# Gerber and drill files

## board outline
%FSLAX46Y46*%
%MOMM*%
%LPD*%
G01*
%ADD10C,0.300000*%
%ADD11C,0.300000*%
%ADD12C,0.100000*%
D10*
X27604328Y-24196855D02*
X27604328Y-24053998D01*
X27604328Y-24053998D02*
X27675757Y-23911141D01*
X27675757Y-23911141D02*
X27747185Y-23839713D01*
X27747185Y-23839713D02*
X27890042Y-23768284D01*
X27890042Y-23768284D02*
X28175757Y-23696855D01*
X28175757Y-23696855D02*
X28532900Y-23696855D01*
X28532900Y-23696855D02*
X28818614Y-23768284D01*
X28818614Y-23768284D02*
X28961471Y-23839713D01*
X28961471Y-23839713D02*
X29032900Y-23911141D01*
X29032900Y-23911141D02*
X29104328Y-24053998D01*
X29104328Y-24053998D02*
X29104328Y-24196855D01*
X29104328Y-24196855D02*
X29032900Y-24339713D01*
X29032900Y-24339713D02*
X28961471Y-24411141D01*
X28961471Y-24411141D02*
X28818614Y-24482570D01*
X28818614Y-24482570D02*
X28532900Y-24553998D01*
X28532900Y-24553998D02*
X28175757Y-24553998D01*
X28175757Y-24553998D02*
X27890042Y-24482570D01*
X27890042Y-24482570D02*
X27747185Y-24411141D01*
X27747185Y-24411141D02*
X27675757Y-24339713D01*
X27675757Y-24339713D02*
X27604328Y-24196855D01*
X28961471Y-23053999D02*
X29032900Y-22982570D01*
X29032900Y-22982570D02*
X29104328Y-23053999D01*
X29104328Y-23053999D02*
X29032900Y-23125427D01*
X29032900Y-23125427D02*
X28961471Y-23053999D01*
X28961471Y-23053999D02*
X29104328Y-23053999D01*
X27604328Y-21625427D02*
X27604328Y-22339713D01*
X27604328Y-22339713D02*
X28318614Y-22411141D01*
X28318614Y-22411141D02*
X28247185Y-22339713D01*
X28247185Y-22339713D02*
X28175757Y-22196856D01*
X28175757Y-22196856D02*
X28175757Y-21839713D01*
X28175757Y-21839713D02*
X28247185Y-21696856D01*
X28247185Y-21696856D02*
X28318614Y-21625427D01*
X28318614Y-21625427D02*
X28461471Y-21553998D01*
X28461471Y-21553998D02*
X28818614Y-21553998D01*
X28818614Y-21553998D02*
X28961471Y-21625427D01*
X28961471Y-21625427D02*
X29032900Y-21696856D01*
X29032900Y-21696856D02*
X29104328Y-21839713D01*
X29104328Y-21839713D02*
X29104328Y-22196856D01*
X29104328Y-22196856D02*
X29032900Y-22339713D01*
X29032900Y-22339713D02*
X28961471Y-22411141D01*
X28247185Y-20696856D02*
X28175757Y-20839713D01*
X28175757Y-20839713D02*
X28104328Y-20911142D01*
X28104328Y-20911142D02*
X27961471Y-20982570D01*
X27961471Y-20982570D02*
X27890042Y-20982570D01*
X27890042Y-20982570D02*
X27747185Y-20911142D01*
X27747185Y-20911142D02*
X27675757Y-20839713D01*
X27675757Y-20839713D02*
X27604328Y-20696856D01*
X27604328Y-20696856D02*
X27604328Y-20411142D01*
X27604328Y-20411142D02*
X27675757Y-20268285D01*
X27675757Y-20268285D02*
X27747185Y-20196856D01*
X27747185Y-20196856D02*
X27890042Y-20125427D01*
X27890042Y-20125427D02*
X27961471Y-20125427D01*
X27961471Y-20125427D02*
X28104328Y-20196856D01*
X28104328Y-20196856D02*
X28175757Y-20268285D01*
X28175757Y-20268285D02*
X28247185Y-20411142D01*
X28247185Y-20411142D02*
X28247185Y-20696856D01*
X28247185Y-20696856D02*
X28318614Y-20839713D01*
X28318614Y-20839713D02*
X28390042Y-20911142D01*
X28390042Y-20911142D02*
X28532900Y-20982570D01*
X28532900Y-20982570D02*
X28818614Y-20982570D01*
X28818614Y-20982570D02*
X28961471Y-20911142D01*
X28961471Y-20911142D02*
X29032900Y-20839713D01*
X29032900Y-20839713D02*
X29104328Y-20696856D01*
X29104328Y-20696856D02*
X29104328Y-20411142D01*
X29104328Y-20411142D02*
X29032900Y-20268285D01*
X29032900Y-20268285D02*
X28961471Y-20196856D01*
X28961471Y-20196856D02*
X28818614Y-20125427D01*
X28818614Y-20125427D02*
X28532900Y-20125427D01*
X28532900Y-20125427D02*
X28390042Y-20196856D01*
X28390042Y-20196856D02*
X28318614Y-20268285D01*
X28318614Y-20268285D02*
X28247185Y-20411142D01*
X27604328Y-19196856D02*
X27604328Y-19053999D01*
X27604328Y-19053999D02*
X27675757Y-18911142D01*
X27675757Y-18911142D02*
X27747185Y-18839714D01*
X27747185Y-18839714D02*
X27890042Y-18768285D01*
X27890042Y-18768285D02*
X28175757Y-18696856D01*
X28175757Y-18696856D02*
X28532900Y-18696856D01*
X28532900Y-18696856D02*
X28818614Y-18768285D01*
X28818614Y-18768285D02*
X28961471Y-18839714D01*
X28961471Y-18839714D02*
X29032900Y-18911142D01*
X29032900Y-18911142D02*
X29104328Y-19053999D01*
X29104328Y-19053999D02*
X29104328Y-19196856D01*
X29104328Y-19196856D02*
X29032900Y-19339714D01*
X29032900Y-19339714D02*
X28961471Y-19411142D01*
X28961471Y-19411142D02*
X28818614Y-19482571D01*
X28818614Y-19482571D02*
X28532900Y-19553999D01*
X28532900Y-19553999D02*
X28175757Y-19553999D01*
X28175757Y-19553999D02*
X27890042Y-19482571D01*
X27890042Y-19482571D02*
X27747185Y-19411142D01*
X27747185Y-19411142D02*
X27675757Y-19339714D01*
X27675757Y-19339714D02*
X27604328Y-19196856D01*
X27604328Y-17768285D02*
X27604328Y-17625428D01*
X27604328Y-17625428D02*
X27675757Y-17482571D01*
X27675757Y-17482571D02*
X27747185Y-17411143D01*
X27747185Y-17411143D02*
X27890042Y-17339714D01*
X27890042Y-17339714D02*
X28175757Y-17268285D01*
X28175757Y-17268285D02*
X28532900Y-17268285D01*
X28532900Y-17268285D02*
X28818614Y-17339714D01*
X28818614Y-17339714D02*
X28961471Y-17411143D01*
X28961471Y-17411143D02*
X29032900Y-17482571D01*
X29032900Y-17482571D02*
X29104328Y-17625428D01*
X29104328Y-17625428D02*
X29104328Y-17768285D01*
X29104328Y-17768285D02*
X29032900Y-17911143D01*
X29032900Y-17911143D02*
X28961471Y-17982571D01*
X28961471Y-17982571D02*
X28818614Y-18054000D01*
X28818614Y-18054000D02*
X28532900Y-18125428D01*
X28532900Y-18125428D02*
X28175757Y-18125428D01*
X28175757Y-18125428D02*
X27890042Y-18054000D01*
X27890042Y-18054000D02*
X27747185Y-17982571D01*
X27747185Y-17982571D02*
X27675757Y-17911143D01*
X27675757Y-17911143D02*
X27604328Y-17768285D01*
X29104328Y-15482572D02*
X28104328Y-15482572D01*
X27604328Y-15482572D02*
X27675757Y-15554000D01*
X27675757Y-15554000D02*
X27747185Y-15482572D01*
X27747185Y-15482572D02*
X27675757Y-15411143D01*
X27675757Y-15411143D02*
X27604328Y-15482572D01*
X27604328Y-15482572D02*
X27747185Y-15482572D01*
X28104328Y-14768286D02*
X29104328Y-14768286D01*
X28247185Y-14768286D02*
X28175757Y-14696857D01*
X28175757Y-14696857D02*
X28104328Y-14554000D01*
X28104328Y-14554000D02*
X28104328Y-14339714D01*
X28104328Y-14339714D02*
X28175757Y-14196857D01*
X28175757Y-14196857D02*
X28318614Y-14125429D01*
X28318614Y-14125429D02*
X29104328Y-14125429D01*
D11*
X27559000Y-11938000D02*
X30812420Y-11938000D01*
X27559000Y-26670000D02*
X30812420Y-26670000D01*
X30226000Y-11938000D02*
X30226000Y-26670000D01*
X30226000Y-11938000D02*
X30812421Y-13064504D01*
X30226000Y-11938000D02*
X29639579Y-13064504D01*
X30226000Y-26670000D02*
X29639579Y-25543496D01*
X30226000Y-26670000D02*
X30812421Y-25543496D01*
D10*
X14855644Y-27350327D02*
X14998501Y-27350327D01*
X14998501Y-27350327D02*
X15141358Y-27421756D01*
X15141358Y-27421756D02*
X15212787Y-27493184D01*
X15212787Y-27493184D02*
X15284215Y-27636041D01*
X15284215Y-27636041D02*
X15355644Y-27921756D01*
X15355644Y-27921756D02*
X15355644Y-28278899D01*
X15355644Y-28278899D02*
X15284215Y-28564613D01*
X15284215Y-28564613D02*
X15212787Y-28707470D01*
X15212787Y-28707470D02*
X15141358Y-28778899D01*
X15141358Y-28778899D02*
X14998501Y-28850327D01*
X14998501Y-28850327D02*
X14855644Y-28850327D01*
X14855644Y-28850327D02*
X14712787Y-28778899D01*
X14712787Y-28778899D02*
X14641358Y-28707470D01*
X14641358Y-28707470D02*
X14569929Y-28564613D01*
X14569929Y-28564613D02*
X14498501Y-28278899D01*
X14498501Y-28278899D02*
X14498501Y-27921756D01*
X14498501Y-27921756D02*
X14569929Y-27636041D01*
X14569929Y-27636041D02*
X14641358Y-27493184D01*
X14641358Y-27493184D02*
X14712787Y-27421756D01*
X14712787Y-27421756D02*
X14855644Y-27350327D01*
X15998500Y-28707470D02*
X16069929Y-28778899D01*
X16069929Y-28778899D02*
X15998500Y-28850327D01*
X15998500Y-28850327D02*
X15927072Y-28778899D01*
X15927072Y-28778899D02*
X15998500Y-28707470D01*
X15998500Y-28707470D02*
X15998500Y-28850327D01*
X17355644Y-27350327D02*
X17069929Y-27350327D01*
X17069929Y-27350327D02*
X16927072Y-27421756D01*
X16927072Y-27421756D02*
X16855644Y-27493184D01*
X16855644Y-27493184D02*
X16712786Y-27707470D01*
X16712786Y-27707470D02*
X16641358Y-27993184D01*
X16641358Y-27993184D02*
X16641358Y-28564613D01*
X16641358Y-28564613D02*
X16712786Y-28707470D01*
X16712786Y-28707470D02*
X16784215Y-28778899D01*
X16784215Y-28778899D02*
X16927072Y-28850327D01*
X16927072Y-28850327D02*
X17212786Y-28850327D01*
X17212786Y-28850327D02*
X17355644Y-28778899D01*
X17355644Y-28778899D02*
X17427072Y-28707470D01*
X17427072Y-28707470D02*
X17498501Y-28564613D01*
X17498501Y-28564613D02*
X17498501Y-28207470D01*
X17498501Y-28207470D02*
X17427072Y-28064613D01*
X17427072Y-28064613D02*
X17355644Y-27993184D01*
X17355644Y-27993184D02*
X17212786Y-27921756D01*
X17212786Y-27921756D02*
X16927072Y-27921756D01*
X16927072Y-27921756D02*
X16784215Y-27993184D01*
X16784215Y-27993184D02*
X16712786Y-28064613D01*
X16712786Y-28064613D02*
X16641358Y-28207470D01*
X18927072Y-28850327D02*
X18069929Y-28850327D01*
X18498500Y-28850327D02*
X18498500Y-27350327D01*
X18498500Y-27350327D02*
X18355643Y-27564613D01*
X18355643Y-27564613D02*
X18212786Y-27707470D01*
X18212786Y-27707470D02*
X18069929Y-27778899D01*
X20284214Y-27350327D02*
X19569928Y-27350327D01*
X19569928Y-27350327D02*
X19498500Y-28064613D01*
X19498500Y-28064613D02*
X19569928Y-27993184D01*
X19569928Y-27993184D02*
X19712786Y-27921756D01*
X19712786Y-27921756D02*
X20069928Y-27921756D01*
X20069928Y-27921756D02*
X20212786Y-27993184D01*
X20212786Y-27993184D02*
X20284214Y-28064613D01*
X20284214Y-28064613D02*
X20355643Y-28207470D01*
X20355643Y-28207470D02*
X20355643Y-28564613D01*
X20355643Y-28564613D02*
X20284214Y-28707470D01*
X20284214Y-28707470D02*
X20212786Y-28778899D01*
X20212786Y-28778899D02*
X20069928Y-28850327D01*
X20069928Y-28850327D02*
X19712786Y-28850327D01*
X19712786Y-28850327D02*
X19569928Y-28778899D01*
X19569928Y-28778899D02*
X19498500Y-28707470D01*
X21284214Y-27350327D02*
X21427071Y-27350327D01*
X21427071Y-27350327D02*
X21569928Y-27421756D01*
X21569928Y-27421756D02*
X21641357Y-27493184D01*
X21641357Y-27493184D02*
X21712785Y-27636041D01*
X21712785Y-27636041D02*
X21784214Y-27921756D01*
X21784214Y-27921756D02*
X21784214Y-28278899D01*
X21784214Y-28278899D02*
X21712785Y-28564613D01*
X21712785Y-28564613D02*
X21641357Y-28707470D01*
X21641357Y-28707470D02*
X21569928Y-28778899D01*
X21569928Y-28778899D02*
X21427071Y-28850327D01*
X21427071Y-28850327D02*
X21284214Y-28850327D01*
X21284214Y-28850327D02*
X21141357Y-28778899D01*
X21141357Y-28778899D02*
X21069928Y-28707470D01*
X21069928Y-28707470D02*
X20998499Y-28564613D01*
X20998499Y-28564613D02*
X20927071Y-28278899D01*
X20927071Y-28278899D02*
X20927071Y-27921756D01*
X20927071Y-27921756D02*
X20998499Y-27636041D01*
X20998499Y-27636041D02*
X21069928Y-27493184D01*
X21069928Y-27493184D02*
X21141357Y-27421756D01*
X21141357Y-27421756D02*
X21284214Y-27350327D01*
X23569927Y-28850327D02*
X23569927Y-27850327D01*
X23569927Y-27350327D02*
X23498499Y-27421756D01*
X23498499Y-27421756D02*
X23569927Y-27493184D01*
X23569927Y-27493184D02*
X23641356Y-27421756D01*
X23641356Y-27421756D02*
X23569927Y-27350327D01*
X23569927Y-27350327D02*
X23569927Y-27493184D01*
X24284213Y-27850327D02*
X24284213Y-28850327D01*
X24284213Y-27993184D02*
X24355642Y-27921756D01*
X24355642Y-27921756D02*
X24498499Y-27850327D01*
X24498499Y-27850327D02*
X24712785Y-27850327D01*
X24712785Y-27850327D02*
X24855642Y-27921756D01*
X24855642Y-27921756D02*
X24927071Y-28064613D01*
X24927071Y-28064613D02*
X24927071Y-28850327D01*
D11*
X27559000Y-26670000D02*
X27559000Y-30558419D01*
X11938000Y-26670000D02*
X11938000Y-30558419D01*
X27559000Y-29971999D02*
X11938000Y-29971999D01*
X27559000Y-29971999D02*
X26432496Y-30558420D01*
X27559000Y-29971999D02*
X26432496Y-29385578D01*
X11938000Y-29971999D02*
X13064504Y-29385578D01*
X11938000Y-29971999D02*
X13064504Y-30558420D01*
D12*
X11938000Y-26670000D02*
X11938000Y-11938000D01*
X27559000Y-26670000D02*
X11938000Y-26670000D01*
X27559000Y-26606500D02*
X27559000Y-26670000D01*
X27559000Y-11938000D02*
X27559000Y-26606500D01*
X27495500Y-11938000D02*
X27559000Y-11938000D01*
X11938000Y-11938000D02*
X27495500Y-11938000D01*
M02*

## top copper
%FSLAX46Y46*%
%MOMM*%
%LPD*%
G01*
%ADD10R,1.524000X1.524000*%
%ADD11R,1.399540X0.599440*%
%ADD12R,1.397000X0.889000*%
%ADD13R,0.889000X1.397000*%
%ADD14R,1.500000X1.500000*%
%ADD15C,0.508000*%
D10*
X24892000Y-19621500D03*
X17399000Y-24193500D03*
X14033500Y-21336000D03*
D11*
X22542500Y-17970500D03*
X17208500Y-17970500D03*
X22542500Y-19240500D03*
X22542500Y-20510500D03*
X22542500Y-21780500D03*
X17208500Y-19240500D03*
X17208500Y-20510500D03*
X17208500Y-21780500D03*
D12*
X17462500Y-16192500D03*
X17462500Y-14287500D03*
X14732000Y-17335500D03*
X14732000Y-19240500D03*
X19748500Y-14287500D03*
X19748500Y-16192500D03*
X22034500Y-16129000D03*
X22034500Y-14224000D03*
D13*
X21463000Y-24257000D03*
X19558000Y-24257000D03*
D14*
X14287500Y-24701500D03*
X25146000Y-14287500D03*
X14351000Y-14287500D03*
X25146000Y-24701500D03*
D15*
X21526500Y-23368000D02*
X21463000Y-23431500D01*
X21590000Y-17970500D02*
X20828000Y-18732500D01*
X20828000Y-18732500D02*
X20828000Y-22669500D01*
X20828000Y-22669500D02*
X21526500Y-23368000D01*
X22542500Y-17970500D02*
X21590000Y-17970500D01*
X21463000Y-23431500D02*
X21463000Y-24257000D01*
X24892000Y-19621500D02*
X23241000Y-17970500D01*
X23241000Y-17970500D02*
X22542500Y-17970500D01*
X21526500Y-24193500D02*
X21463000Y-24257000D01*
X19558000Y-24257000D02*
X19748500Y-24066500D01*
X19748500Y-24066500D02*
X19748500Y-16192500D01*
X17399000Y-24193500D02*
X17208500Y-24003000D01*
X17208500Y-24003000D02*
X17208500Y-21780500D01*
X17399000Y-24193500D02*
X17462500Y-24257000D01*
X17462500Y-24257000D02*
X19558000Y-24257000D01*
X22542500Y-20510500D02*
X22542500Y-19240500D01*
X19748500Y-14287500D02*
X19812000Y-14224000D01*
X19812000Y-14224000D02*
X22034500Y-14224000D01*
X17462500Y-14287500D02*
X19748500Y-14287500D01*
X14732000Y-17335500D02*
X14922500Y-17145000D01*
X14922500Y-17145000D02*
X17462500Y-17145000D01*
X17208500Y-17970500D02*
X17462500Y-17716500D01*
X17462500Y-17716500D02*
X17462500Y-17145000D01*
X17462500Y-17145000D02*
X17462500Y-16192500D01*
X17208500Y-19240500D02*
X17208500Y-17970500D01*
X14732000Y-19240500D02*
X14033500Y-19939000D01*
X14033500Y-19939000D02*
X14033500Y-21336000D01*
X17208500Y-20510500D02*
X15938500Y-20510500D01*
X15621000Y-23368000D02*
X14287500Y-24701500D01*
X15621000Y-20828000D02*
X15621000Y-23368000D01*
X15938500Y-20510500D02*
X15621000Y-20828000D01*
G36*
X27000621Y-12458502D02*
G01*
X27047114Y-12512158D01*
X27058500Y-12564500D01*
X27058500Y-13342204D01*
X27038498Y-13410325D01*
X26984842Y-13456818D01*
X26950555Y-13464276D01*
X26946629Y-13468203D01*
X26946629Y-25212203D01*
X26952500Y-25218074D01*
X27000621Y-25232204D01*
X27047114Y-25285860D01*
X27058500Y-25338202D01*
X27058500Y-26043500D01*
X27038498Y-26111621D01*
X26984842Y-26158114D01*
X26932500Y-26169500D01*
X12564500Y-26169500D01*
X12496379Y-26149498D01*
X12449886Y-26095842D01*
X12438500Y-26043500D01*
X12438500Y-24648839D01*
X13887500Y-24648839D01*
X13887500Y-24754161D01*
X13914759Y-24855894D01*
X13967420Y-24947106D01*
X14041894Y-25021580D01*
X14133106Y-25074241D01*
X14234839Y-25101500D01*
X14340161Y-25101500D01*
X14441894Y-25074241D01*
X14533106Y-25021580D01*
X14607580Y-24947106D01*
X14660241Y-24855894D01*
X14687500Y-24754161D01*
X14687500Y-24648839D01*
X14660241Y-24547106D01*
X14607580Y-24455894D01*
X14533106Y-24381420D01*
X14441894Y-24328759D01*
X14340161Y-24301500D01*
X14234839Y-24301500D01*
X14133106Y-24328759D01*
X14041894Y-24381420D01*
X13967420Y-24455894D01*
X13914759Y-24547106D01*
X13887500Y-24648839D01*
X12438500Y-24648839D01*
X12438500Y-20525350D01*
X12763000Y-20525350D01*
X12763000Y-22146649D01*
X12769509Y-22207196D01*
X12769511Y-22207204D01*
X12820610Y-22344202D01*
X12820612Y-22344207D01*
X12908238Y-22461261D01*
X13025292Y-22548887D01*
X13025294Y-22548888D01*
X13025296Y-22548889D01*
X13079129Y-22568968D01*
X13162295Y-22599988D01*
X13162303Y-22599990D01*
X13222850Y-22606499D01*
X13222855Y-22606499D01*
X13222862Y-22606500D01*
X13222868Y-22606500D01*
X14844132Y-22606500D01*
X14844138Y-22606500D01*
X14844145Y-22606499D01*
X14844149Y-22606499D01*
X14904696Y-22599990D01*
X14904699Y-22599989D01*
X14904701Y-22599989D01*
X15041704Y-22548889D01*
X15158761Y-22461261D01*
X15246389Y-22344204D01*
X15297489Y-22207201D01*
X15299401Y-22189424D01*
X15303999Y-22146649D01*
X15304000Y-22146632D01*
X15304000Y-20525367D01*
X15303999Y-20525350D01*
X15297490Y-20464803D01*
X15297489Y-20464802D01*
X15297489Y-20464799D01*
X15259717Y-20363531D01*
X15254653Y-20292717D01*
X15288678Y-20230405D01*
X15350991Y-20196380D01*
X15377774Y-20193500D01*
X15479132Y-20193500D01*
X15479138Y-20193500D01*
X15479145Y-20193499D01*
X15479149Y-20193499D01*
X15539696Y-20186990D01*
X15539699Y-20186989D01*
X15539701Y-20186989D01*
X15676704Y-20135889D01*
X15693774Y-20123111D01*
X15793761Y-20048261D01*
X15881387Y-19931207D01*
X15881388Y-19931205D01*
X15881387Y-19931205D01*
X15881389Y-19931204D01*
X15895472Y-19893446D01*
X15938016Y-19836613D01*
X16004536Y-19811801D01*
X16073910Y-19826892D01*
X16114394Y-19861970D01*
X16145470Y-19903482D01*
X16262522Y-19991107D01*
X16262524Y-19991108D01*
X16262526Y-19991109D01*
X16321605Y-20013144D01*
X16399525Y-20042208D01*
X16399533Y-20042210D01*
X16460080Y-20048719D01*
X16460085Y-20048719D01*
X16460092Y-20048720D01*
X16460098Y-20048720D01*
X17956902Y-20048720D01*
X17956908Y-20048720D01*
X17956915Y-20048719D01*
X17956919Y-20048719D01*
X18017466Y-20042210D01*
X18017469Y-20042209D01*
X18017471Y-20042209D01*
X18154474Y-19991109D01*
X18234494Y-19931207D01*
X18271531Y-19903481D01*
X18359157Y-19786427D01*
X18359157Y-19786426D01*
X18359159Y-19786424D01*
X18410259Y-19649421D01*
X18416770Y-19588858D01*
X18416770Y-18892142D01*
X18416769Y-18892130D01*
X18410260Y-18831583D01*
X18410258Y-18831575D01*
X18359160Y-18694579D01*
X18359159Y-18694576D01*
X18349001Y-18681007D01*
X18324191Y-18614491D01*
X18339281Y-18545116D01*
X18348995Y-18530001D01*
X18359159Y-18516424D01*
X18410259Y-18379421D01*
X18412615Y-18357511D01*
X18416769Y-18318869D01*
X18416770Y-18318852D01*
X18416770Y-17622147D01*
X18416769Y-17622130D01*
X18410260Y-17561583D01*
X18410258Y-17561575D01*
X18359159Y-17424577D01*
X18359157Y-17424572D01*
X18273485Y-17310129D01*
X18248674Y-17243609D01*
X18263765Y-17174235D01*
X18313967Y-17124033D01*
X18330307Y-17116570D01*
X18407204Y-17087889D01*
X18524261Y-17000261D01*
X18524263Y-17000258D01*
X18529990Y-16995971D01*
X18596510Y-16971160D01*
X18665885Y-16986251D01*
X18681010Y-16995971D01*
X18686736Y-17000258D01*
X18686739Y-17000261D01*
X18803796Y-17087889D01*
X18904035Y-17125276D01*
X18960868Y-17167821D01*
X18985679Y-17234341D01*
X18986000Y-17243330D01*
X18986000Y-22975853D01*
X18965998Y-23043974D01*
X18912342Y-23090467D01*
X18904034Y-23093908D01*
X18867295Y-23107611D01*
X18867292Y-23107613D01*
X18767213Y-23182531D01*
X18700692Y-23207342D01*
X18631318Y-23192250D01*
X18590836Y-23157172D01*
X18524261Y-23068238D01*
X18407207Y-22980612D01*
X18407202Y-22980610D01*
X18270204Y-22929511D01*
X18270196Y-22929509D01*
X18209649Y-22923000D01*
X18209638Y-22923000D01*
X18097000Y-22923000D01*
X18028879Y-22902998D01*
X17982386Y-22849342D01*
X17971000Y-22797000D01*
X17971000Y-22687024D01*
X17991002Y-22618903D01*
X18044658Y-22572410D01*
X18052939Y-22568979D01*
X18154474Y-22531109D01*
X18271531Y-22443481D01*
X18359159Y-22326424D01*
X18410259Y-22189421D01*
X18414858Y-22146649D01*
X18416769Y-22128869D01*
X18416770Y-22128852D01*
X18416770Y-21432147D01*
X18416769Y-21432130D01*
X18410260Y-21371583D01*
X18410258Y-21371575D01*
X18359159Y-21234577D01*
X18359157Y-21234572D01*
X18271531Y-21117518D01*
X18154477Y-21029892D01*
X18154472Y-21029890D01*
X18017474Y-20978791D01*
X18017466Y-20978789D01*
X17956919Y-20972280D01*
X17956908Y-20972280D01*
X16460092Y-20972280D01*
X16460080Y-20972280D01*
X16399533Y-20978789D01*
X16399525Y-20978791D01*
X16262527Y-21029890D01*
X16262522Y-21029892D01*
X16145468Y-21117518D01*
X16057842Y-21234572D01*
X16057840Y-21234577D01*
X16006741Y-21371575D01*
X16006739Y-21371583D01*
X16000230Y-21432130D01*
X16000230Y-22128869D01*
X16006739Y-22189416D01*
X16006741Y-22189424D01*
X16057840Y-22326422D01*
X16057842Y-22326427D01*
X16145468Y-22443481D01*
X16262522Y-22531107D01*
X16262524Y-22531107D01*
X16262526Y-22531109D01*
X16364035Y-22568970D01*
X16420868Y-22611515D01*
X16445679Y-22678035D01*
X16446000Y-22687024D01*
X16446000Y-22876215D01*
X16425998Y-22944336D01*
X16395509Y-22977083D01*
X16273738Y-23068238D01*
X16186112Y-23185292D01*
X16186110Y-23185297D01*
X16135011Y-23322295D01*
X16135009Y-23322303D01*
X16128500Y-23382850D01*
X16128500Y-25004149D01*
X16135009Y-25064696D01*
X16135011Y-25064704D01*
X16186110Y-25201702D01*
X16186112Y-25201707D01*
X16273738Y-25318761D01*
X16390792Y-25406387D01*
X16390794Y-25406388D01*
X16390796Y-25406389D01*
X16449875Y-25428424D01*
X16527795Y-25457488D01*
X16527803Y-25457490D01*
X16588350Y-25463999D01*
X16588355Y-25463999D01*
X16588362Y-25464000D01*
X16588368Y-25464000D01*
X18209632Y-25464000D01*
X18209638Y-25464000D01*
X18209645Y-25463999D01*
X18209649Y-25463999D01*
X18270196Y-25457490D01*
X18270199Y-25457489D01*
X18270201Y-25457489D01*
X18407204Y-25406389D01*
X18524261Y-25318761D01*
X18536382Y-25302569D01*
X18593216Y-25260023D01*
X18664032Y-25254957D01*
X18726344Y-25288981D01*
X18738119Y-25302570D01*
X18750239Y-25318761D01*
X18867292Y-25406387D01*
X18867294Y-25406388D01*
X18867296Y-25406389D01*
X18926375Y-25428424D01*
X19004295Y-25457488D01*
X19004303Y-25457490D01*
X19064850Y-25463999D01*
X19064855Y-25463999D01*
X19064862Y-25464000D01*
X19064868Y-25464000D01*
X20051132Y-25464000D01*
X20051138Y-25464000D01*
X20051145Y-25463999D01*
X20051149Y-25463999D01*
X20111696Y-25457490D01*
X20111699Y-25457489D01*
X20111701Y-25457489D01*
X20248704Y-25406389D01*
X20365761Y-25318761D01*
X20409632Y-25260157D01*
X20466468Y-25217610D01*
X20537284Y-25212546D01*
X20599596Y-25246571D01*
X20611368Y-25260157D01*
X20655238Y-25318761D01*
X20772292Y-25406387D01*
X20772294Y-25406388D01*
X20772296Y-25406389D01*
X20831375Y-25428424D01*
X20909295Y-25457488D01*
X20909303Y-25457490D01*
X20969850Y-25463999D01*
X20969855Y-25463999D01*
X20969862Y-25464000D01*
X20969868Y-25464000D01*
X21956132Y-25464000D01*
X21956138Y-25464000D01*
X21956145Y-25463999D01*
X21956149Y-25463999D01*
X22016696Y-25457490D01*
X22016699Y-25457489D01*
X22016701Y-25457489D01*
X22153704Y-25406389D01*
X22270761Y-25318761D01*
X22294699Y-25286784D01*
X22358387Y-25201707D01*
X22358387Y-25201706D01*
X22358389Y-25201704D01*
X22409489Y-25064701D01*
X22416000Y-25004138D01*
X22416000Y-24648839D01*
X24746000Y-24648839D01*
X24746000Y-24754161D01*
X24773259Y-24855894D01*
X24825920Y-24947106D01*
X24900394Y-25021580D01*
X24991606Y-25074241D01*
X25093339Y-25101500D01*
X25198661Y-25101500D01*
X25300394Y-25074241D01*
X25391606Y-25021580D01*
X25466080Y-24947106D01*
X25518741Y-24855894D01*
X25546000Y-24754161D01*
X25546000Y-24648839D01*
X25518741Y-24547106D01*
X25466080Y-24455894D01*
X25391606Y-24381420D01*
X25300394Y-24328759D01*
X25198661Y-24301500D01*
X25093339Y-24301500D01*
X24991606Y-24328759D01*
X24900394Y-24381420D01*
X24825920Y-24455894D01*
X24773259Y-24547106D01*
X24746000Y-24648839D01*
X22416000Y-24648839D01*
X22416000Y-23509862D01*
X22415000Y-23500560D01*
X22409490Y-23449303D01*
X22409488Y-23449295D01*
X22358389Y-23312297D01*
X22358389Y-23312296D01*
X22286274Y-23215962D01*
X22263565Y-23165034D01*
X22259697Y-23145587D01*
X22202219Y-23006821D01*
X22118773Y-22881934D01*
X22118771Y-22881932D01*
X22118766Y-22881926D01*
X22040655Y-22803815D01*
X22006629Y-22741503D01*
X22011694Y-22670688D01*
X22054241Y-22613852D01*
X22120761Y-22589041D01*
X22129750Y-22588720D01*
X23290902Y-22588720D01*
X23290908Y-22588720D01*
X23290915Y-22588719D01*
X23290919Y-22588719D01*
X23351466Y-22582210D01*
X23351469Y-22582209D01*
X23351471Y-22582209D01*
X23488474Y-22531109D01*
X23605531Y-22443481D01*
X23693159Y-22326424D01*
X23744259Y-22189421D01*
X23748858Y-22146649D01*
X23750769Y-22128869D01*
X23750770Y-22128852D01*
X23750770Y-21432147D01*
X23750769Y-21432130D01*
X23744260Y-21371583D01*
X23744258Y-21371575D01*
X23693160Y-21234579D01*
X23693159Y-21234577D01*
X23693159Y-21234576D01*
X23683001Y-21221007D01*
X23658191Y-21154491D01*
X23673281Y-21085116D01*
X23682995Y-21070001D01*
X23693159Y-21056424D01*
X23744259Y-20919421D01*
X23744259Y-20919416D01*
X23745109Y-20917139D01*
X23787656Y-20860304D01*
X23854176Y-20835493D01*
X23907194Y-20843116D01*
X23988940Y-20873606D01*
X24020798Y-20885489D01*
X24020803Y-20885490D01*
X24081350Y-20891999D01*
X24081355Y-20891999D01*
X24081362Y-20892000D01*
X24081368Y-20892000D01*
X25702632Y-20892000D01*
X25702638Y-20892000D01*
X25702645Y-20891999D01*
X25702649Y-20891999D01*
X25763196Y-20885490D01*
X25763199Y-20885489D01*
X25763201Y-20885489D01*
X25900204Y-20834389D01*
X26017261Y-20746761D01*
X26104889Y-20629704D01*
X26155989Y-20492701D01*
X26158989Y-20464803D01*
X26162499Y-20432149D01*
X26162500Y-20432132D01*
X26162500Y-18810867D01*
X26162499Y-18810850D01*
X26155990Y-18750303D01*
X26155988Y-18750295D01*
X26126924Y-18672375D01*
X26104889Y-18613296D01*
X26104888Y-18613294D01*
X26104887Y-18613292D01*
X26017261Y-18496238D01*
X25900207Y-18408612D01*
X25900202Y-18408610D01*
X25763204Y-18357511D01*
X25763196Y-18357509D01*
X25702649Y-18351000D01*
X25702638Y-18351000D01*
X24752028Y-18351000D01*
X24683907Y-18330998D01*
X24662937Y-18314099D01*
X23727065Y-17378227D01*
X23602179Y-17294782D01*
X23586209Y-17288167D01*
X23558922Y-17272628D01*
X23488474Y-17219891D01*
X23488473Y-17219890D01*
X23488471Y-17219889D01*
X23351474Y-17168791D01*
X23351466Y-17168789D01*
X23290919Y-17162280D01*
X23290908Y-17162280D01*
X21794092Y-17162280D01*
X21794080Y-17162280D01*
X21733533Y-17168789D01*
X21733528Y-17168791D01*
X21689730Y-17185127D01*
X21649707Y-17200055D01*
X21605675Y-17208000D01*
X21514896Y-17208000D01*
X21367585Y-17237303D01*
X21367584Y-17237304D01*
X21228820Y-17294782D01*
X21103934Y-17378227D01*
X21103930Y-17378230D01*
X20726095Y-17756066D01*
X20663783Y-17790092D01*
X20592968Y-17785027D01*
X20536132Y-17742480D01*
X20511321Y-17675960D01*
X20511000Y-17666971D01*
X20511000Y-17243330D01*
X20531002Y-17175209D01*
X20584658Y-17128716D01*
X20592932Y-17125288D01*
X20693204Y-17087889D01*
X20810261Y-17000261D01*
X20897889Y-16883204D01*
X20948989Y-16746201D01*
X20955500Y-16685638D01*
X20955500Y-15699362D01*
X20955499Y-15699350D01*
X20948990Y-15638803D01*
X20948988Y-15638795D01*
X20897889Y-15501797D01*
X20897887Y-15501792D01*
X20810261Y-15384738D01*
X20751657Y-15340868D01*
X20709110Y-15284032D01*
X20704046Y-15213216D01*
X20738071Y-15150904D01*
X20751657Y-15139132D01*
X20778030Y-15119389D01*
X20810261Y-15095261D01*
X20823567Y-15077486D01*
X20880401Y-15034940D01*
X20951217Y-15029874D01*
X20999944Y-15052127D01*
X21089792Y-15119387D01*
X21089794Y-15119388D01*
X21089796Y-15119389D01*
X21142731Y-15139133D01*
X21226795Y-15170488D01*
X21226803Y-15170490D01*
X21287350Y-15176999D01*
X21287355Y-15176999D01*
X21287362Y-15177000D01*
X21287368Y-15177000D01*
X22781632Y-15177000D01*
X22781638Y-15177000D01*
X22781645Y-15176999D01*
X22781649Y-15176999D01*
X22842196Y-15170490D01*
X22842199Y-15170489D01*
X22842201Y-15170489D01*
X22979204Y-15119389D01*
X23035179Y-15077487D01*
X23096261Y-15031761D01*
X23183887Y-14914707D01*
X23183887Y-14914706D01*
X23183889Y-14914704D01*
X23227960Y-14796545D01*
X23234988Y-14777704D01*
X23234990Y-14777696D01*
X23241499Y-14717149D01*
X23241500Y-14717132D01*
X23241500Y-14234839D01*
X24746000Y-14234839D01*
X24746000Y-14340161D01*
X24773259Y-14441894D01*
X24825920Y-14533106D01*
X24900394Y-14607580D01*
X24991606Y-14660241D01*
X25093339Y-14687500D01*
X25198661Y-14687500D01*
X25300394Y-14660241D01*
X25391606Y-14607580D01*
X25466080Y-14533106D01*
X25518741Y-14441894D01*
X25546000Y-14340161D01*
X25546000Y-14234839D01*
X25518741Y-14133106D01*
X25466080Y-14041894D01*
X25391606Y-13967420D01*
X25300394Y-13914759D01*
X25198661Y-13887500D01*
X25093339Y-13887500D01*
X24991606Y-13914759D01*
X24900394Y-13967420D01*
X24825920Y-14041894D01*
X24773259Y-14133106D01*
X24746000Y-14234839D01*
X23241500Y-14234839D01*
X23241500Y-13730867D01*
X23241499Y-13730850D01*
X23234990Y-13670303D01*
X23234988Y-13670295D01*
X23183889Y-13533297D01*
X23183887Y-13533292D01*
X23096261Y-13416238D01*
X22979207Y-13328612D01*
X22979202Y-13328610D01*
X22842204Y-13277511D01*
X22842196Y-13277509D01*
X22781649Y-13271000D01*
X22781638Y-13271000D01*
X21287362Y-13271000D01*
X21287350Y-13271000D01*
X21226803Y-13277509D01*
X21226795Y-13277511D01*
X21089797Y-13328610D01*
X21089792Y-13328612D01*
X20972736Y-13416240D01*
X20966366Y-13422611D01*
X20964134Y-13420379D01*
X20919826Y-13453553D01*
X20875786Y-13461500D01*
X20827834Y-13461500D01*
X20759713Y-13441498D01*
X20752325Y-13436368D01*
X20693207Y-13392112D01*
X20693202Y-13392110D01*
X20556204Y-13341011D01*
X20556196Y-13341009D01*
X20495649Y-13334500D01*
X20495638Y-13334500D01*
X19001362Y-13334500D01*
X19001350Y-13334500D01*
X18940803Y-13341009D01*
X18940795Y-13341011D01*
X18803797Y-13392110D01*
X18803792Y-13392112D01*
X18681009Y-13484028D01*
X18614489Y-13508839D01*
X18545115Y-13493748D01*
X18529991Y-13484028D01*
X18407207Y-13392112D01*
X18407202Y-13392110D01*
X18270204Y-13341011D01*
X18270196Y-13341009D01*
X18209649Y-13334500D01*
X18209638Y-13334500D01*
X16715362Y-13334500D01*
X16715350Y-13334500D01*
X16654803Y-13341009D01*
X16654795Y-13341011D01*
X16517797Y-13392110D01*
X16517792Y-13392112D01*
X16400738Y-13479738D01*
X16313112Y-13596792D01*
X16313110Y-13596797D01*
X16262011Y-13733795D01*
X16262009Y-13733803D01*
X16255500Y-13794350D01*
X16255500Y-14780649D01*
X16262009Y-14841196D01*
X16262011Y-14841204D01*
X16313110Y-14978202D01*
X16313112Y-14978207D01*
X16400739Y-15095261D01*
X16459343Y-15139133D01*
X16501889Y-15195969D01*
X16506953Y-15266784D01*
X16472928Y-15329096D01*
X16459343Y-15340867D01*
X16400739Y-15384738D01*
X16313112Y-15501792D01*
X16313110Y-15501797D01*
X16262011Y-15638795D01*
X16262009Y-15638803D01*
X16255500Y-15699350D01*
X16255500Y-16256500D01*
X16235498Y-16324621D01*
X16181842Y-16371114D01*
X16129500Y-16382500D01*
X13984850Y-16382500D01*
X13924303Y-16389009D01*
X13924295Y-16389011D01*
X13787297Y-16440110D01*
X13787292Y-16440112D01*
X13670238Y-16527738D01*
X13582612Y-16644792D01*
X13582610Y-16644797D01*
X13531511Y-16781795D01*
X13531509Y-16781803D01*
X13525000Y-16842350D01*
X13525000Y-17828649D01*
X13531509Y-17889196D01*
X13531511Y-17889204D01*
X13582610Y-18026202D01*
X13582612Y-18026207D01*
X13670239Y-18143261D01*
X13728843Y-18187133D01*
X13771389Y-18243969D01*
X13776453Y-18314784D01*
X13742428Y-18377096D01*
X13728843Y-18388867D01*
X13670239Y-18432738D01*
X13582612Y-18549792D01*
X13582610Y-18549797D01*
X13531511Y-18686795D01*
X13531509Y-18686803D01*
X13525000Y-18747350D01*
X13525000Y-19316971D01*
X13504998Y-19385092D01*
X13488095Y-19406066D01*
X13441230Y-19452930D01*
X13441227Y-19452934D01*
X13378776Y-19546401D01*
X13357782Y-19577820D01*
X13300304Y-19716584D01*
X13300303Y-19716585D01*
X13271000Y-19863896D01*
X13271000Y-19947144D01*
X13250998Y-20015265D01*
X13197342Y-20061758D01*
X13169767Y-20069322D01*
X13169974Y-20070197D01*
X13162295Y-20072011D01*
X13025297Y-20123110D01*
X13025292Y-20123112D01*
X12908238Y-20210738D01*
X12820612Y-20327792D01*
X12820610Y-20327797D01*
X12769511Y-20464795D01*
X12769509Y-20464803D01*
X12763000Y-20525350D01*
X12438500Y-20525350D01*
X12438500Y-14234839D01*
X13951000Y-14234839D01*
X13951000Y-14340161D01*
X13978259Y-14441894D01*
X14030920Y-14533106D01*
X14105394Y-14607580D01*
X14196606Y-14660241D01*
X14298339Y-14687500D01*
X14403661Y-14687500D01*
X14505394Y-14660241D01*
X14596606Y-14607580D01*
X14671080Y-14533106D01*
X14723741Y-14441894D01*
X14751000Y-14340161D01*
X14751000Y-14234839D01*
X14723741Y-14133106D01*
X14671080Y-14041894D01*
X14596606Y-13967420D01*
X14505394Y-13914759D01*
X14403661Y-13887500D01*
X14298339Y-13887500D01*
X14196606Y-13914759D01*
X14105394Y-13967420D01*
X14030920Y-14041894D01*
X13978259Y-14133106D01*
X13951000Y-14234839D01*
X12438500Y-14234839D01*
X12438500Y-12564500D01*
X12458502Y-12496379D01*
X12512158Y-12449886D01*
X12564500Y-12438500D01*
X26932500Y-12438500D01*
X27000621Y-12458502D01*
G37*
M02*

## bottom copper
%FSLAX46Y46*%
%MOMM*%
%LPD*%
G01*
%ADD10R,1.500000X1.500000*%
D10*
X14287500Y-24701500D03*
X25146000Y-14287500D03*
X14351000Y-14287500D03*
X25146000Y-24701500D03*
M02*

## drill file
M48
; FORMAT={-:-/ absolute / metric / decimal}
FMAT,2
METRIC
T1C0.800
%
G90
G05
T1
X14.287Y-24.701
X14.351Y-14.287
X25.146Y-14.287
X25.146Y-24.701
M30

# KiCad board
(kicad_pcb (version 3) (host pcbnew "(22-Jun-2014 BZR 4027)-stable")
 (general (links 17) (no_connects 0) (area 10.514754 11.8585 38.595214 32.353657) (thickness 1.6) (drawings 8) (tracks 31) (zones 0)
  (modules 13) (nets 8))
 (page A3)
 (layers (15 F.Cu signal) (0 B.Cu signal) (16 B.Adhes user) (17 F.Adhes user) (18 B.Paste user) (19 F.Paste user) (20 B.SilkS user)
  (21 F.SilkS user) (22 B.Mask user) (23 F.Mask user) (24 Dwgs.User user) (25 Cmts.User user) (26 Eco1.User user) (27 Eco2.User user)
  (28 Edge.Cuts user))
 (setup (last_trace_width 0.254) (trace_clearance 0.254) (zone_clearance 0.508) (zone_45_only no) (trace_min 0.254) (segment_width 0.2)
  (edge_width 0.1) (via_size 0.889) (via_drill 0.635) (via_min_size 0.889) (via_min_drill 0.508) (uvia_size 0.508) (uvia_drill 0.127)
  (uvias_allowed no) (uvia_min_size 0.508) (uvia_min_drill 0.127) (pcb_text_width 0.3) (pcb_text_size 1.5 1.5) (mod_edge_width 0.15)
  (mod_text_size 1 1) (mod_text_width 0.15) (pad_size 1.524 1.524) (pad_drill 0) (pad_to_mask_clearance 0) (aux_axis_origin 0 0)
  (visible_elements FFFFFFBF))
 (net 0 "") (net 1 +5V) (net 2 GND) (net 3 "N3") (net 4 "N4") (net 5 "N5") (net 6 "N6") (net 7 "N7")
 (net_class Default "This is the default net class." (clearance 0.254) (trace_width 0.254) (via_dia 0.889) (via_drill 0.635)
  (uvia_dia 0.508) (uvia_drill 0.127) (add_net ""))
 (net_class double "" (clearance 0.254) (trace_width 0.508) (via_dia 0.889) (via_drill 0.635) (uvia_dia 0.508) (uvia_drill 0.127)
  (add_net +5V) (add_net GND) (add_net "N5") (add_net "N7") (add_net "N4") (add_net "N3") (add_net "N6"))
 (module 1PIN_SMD (layer F.Cu) (at 24.892 19.6215)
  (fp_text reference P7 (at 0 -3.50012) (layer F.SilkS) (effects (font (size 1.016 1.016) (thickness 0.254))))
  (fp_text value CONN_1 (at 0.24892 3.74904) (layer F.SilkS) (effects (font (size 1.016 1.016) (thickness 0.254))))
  (pad 1 smd rect (at 0 0) (size 1.524 1.524) (layers F.Cu F.Paste F.SilkS F.Mask) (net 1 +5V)))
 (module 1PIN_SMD (layer F.Cu) (at 17.399 24.1935)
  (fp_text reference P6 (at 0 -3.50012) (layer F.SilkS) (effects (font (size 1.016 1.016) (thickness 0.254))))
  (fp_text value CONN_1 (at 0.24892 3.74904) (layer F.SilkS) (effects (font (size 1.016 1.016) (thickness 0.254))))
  (pad 1 smd rect (at 0 0) (size 1.524 1.524) (layers F.Cu F.Paste F.SilkS F.Mask) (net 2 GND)))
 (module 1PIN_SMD (layer F.Cu) (at 14.0335 21.336)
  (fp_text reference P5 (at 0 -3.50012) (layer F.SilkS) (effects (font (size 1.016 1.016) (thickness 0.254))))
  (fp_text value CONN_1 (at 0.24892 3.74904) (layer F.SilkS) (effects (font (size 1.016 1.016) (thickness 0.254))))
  (pad 1 smd rect (at 0 0) (size 1.524 1.524) (layers F.Cu F.Paste F.SilkS F.Mask) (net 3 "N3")))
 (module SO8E (layer F.Cu) (at 19.8755 19.8755 270)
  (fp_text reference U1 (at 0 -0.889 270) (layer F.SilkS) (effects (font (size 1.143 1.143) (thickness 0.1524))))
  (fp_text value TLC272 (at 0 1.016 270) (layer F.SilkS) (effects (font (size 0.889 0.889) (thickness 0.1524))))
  (pad 8 smd rect (at -1.905 -2.667 270) (size 0.59944 1.39954) (layers F.Cu F.Paste F.Mask) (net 1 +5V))
  (pad 1 smd rect (at -1.905 2.667 270) (size 0.59944 1.39954) (layers F.Cu F.Paste F.Mask) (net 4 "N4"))
  (pad 7 smd rect (at -0.635 -2.667 270) (size 0.59944 1.39954) (layers F.Cu F.Paste F.Mask) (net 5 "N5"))
  (pad 6 smd rect (at 0.635 -2.667 270) (size 0.59944 1.39954) (layers F.Cu F.Paste F.Mask) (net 5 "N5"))
  (pad 5 smd rect (at 1.905 -2.667 270) (size 0.59944 1.39954) (layers F.Cu F.Paste F.Mask))
  (pad 2 smd rect (at -0.635 2.667 270) (size 0.59944 1.39954) (layers F.Cu F.Paste F.Mask) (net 4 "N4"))
  (pad 3 smd rect (at 0.635 2.667 270) (size 0.59944 1.39954) (layers F.Cu F.Paste F.Mask) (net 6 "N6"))
  (pad 4 smd rect (at 1.905 2.667 270) (size 0.59944 1.39954) (layers F.Cu F.Paste F.Mask) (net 2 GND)))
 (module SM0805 (layer F.Cu) (at 17.4625 15.24 90)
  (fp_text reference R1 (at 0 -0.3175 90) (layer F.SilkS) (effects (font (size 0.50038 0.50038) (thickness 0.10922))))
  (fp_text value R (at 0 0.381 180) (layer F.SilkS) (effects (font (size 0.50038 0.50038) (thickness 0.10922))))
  (pad 1 smd rect (at -0.9525 0 90) (size 0.889 1.397) (layers F.Cu F.Paste F.Mask) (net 4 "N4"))
  (pad 2 smd rect (at 0.9525 0 90) (size 0.889 1.397) (layers F.Cu F.Paste F.Mask) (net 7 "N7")))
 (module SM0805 (layer F.Cu) (at 14.732 18.288 270)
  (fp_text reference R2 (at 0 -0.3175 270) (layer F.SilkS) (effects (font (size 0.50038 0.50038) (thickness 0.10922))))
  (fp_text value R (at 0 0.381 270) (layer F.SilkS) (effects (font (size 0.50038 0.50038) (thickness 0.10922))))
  (pad 1 smd rect (at -0.9525 0 270) (size 0.889 1.397) (layers F.Cu F.Paste F.Mask) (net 4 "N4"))
  (pad 2 smd rect (at 0.9525 0 270) (size 0.889 1.397) (layers F.Cu F.Paste F.Mask) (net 3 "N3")))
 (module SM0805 (layer F.Cu) (at 19.7485 15.24 270)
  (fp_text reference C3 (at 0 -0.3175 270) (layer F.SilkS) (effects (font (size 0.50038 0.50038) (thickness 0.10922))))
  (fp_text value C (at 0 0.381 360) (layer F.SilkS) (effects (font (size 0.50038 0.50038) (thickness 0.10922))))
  (pad 1 smd rect (at -0.9525 0 270) (size 0.889 1.397) (layers F.Cu F.Paste F.Mask) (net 7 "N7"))
  (pad 2 smd rect (at 0.9525 0 270) (size 0.889 1.397) (layers F.Cu F.Paste F.Mask) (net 2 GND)))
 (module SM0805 (layer F.Cu) (at 22.0345 15.1765 90)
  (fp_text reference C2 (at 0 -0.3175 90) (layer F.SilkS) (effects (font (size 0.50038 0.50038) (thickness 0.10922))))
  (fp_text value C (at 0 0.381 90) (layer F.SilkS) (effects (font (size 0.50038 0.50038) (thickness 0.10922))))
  (pad 1 smd rect (at -0.9525 0 90) (size 0.889 1.397) (layers F.Cu F.Paste F.Mask) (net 6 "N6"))
  (pad 2 smd rect (at 0.9525 0 90) (size 0.889 1.397) (layers F.Cu F.Paste F.Mask) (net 7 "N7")))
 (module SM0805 (layer F.Cu) (at 20.5105 24.257 180)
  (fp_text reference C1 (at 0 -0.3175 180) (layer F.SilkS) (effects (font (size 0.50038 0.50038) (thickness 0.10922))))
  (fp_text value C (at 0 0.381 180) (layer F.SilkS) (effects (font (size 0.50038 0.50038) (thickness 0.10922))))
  (pad 1 smd rect (at -0.9525 0 180) (size 0.889 1.397) (layers F.Cu F.Paste F.Mask) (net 1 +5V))
  (pad 2 smd rect (at 0.9525 0 180) (size 0.889 1.397) (layers F.Cu F.Paste F.Mask) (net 2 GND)))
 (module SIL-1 (layer F.Cu) (at 14.2875 24.7015)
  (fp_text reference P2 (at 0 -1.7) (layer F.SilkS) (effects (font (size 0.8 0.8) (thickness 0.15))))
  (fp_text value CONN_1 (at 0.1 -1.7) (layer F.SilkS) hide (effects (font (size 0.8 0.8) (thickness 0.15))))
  (pad 1 thru_hole rect (at 0 0) (size 1.5 1.5) (drill 0.8) (layers *.Cu *.Mask F.SilkS) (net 6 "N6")))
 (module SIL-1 (layer F.Cu) (at 25.146 14.2875)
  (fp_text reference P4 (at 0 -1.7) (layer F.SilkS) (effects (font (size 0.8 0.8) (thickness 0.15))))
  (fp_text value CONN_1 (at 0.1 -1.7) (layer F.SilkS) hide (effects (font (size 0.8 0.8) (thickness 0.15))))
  (pad 1 thru_hole rect (at 0 0) (size 1.5 1.5) (drill 0.8) (layers *.Cu *.Mask F.SilkS) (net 6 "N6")))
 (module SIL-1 (layer F.Cu) (at 14.351 14.2875)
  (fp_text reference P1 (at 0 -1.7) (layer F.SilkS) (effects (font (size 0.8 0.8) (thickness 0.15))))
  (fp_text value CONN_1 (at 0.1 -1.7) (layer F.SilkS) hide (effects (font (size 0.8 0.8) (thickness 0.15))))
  (pad 1 thru_hole rect (at 0 0) (size 1.5 1.5) (drill 0.8) (layers *.Cu *.Mask F.SilkS) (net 6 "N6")))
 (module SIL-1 (layer F.Cu) (at 25.146 24.7015)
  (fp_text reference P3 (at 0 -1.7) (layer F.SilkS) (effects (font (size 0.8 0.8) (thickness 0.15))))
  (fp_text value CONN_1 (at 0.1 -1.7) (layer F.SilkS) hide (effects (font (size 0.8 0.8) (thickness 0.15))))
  (pad 1 thru_hole rect (at 0 0) (size 1.5 1.5) (drill 0.8) (layers *.Cu *.Mask F.SilkS) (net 6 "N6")))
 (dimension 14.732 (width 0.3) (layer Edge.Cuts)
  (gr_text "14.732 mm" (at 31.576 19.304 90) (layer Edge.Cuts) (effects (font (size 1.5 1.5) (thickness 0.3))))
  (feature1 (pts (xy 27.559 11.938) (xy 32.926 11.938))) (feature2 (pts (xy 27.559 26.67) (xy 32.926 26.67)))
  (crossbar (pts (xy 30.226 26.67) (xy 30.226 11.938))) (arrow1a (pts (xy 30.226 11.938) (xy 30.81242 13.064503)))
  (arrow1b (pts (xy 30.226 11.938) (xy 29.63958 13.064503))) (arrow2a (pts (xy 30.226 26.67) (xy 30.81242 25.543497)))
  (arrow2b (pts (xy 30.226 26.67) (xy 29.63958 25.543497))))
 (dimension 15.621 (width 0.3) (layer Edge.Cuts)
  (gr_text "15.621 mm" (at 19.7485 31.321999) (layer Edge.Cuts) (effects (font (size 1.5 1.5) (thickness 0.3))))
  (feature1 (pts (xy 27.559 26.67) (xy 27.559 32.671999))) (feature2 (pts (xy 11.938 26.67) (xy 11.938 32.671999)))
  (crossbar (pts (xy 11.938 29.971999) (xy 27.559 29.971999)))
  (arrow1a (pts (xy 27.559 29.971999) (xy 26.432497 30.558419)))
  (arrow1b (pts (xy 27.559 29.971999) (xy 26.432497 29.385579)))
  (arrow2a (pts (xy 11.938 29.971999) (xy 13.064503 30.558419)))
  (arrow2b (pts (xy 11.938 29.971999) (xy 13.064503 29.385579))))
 (gr_line (start 11.938 26.67) (end 11.938 11.938) (angle 90) (layer Edge.Cuts) (width 0.1))
 (gr_line (start 27.559 26.67) (end 11.938 26.67) (angle 90) (layer Edge.Cuts) (width 0.1))
 (gr_line (start 27.559 26.6065) (end 27.559 26.67) (angle 90) (layer Edge.Cuts) (width 0.1))
 (gr_line (start 27.559 11.938) (end 27.559 26.6065) (angle 90) (layer Edge.Cuts) (width 0.1))
 (gr_line (start 27.4955 11.938) (end 27.559 11.938) (angle 90) (layer Edge.Cuts) (width 0.1))
 (gr_line (start 11.938 11.938) (end 27.4955 11.938) (angle 90) (layer Edge.Cuts) (width 0.1))
 (segment (start 21.5265 23.368) (end 21.463 23.4315) (width 0.508) (layer F.Cu) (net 1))
 (segment (start 21.59 17.9705) (end 20.828 18.7325) (width 0.508) (layer F.Cu) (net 1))
 (segment (start 20.828 18.7325) (end 20.828 22.6695) (width 0.508) (layer F.Cu) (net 1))
 (segment (start 20.828 22.6695) (end 21.5265 23.368) (width 0.508) (layer F.Cu) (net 1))
 (segment (start 22.5425 17.9705) (end 21.59 17.9705) (width 0.508) (layer F.Cu) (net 1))
 (segment (start 21.463 23.4315) (end 21.463 24.257) (width 0.508) (layer F.Cu) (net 1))
 (segment (start 24.892 19.6215) (end 23.241 17.9705) (width 0.508) (layer F.Cu) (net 1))
 (segment (start 23.241 17.9705) (end 22.5425 17.9705) (width 0.508) (layer F.Cu) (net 1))
 (segment (start 21.5265 24.1935) (end 21.463 24.257) (width 0.508) (layer F.Cu) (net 1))
 (segment (start 19.558 24.257) (end 19.7485 24.0665) (width 0.508) (layer F.Cu) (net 2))
 (segment (start 19.7485 24.0665) (end 19.7485 16.1925) (width 0.508) (layer F.Cu) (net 2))
 (segment (start 17.399 24.1935) (end 17.2085 24.003) (width 0.508) (layer F.Cu) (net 2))
 (segment (start 17.2085 24.003) (end 17.2085 21.7805) (width 0.508) (layer F.Cu) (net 2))
 (segment (start 17.399 24.1935) (end 17.4625 24.257) (width 0.508) (layer F.Cu) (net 2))
 (segment (start 17.4625 24.257) (end 19.558 24.257) (width 0.508) (layer F.Cu) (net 2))
 (segment (start 22.5425 20.5105) (end 22.5425 19.2405) (width 0.508) (layer F.Cu) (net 5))
 (segment (start 19.7485 14.2875) (end 19.812 14.224) (width 0.508) (layer F.Cu) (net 7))
 (segment (start 19.812 14.224) (end 22.0345 14.224) (width 0.508) (layer F.Cu) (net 7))
 (segment (start 17.4625 14.2875) (end 19.7485 14.2875) (width 0.508) (layer F.Cu) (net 7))
 (segment (start 14.732 17.3355) (end 14.9225 17.145) (width 0.508) (layer F.Cu) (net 4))
 (segment (start 14.9225 17.145) (end 17.4625 17.145) (width 0.508) (layer F.Cu) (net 4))
 (segment (start 17.2085 17.9705) (end 17.4625 17.7165) (width 0.508) (layer F.Cu) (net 4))
 (segment (start 17.4625 17.7165) (end 17.4625 17.145) (width 0.508) (layer F.Cu) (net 4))
 (segment (start 17.4625 17.145) (end 17.4625 16.1925) (width 0.508) (layer F.Cu) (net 4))
 (segment (start 17.2085 19.2405) (end 17.2085 17.9705) (width 0.508) (layer F.Cu) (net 4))
 (segment (start 14.732 19.2405) (end 14.0335 19.939) (width 0.508) (layer F.Cu) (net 3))
 (segment (start 14.0335 19.939) (end 14.0335 21.336) (width 0.508) (layer F.Cu) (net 3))
 (segment (start 17.2085 20.5105) (end 15.9385 20.5105) (width 0.508) (layer F.Cu) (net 6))
 (segment (start 15.621 23.368) (end 14.2875 24.7015) (width 0.508) (layer F.Cu) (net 6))
 (segment (start 15.621 20.828) (end 15.621 23.368) (width 0.508) (layer F.Cu) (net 6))
 (segment (start 15.9385 20.5105) (end 15.621 20.828) (width 0.508) (layer F.Cu) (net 6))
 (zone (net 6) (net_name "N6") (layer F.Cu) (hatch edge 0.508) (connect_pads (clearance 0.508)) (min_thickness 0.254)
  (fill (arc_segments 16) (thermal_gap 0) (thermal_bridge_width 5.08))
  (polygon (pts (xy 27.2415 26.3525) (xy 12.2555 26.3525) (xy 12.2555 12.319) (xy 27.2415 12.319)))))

